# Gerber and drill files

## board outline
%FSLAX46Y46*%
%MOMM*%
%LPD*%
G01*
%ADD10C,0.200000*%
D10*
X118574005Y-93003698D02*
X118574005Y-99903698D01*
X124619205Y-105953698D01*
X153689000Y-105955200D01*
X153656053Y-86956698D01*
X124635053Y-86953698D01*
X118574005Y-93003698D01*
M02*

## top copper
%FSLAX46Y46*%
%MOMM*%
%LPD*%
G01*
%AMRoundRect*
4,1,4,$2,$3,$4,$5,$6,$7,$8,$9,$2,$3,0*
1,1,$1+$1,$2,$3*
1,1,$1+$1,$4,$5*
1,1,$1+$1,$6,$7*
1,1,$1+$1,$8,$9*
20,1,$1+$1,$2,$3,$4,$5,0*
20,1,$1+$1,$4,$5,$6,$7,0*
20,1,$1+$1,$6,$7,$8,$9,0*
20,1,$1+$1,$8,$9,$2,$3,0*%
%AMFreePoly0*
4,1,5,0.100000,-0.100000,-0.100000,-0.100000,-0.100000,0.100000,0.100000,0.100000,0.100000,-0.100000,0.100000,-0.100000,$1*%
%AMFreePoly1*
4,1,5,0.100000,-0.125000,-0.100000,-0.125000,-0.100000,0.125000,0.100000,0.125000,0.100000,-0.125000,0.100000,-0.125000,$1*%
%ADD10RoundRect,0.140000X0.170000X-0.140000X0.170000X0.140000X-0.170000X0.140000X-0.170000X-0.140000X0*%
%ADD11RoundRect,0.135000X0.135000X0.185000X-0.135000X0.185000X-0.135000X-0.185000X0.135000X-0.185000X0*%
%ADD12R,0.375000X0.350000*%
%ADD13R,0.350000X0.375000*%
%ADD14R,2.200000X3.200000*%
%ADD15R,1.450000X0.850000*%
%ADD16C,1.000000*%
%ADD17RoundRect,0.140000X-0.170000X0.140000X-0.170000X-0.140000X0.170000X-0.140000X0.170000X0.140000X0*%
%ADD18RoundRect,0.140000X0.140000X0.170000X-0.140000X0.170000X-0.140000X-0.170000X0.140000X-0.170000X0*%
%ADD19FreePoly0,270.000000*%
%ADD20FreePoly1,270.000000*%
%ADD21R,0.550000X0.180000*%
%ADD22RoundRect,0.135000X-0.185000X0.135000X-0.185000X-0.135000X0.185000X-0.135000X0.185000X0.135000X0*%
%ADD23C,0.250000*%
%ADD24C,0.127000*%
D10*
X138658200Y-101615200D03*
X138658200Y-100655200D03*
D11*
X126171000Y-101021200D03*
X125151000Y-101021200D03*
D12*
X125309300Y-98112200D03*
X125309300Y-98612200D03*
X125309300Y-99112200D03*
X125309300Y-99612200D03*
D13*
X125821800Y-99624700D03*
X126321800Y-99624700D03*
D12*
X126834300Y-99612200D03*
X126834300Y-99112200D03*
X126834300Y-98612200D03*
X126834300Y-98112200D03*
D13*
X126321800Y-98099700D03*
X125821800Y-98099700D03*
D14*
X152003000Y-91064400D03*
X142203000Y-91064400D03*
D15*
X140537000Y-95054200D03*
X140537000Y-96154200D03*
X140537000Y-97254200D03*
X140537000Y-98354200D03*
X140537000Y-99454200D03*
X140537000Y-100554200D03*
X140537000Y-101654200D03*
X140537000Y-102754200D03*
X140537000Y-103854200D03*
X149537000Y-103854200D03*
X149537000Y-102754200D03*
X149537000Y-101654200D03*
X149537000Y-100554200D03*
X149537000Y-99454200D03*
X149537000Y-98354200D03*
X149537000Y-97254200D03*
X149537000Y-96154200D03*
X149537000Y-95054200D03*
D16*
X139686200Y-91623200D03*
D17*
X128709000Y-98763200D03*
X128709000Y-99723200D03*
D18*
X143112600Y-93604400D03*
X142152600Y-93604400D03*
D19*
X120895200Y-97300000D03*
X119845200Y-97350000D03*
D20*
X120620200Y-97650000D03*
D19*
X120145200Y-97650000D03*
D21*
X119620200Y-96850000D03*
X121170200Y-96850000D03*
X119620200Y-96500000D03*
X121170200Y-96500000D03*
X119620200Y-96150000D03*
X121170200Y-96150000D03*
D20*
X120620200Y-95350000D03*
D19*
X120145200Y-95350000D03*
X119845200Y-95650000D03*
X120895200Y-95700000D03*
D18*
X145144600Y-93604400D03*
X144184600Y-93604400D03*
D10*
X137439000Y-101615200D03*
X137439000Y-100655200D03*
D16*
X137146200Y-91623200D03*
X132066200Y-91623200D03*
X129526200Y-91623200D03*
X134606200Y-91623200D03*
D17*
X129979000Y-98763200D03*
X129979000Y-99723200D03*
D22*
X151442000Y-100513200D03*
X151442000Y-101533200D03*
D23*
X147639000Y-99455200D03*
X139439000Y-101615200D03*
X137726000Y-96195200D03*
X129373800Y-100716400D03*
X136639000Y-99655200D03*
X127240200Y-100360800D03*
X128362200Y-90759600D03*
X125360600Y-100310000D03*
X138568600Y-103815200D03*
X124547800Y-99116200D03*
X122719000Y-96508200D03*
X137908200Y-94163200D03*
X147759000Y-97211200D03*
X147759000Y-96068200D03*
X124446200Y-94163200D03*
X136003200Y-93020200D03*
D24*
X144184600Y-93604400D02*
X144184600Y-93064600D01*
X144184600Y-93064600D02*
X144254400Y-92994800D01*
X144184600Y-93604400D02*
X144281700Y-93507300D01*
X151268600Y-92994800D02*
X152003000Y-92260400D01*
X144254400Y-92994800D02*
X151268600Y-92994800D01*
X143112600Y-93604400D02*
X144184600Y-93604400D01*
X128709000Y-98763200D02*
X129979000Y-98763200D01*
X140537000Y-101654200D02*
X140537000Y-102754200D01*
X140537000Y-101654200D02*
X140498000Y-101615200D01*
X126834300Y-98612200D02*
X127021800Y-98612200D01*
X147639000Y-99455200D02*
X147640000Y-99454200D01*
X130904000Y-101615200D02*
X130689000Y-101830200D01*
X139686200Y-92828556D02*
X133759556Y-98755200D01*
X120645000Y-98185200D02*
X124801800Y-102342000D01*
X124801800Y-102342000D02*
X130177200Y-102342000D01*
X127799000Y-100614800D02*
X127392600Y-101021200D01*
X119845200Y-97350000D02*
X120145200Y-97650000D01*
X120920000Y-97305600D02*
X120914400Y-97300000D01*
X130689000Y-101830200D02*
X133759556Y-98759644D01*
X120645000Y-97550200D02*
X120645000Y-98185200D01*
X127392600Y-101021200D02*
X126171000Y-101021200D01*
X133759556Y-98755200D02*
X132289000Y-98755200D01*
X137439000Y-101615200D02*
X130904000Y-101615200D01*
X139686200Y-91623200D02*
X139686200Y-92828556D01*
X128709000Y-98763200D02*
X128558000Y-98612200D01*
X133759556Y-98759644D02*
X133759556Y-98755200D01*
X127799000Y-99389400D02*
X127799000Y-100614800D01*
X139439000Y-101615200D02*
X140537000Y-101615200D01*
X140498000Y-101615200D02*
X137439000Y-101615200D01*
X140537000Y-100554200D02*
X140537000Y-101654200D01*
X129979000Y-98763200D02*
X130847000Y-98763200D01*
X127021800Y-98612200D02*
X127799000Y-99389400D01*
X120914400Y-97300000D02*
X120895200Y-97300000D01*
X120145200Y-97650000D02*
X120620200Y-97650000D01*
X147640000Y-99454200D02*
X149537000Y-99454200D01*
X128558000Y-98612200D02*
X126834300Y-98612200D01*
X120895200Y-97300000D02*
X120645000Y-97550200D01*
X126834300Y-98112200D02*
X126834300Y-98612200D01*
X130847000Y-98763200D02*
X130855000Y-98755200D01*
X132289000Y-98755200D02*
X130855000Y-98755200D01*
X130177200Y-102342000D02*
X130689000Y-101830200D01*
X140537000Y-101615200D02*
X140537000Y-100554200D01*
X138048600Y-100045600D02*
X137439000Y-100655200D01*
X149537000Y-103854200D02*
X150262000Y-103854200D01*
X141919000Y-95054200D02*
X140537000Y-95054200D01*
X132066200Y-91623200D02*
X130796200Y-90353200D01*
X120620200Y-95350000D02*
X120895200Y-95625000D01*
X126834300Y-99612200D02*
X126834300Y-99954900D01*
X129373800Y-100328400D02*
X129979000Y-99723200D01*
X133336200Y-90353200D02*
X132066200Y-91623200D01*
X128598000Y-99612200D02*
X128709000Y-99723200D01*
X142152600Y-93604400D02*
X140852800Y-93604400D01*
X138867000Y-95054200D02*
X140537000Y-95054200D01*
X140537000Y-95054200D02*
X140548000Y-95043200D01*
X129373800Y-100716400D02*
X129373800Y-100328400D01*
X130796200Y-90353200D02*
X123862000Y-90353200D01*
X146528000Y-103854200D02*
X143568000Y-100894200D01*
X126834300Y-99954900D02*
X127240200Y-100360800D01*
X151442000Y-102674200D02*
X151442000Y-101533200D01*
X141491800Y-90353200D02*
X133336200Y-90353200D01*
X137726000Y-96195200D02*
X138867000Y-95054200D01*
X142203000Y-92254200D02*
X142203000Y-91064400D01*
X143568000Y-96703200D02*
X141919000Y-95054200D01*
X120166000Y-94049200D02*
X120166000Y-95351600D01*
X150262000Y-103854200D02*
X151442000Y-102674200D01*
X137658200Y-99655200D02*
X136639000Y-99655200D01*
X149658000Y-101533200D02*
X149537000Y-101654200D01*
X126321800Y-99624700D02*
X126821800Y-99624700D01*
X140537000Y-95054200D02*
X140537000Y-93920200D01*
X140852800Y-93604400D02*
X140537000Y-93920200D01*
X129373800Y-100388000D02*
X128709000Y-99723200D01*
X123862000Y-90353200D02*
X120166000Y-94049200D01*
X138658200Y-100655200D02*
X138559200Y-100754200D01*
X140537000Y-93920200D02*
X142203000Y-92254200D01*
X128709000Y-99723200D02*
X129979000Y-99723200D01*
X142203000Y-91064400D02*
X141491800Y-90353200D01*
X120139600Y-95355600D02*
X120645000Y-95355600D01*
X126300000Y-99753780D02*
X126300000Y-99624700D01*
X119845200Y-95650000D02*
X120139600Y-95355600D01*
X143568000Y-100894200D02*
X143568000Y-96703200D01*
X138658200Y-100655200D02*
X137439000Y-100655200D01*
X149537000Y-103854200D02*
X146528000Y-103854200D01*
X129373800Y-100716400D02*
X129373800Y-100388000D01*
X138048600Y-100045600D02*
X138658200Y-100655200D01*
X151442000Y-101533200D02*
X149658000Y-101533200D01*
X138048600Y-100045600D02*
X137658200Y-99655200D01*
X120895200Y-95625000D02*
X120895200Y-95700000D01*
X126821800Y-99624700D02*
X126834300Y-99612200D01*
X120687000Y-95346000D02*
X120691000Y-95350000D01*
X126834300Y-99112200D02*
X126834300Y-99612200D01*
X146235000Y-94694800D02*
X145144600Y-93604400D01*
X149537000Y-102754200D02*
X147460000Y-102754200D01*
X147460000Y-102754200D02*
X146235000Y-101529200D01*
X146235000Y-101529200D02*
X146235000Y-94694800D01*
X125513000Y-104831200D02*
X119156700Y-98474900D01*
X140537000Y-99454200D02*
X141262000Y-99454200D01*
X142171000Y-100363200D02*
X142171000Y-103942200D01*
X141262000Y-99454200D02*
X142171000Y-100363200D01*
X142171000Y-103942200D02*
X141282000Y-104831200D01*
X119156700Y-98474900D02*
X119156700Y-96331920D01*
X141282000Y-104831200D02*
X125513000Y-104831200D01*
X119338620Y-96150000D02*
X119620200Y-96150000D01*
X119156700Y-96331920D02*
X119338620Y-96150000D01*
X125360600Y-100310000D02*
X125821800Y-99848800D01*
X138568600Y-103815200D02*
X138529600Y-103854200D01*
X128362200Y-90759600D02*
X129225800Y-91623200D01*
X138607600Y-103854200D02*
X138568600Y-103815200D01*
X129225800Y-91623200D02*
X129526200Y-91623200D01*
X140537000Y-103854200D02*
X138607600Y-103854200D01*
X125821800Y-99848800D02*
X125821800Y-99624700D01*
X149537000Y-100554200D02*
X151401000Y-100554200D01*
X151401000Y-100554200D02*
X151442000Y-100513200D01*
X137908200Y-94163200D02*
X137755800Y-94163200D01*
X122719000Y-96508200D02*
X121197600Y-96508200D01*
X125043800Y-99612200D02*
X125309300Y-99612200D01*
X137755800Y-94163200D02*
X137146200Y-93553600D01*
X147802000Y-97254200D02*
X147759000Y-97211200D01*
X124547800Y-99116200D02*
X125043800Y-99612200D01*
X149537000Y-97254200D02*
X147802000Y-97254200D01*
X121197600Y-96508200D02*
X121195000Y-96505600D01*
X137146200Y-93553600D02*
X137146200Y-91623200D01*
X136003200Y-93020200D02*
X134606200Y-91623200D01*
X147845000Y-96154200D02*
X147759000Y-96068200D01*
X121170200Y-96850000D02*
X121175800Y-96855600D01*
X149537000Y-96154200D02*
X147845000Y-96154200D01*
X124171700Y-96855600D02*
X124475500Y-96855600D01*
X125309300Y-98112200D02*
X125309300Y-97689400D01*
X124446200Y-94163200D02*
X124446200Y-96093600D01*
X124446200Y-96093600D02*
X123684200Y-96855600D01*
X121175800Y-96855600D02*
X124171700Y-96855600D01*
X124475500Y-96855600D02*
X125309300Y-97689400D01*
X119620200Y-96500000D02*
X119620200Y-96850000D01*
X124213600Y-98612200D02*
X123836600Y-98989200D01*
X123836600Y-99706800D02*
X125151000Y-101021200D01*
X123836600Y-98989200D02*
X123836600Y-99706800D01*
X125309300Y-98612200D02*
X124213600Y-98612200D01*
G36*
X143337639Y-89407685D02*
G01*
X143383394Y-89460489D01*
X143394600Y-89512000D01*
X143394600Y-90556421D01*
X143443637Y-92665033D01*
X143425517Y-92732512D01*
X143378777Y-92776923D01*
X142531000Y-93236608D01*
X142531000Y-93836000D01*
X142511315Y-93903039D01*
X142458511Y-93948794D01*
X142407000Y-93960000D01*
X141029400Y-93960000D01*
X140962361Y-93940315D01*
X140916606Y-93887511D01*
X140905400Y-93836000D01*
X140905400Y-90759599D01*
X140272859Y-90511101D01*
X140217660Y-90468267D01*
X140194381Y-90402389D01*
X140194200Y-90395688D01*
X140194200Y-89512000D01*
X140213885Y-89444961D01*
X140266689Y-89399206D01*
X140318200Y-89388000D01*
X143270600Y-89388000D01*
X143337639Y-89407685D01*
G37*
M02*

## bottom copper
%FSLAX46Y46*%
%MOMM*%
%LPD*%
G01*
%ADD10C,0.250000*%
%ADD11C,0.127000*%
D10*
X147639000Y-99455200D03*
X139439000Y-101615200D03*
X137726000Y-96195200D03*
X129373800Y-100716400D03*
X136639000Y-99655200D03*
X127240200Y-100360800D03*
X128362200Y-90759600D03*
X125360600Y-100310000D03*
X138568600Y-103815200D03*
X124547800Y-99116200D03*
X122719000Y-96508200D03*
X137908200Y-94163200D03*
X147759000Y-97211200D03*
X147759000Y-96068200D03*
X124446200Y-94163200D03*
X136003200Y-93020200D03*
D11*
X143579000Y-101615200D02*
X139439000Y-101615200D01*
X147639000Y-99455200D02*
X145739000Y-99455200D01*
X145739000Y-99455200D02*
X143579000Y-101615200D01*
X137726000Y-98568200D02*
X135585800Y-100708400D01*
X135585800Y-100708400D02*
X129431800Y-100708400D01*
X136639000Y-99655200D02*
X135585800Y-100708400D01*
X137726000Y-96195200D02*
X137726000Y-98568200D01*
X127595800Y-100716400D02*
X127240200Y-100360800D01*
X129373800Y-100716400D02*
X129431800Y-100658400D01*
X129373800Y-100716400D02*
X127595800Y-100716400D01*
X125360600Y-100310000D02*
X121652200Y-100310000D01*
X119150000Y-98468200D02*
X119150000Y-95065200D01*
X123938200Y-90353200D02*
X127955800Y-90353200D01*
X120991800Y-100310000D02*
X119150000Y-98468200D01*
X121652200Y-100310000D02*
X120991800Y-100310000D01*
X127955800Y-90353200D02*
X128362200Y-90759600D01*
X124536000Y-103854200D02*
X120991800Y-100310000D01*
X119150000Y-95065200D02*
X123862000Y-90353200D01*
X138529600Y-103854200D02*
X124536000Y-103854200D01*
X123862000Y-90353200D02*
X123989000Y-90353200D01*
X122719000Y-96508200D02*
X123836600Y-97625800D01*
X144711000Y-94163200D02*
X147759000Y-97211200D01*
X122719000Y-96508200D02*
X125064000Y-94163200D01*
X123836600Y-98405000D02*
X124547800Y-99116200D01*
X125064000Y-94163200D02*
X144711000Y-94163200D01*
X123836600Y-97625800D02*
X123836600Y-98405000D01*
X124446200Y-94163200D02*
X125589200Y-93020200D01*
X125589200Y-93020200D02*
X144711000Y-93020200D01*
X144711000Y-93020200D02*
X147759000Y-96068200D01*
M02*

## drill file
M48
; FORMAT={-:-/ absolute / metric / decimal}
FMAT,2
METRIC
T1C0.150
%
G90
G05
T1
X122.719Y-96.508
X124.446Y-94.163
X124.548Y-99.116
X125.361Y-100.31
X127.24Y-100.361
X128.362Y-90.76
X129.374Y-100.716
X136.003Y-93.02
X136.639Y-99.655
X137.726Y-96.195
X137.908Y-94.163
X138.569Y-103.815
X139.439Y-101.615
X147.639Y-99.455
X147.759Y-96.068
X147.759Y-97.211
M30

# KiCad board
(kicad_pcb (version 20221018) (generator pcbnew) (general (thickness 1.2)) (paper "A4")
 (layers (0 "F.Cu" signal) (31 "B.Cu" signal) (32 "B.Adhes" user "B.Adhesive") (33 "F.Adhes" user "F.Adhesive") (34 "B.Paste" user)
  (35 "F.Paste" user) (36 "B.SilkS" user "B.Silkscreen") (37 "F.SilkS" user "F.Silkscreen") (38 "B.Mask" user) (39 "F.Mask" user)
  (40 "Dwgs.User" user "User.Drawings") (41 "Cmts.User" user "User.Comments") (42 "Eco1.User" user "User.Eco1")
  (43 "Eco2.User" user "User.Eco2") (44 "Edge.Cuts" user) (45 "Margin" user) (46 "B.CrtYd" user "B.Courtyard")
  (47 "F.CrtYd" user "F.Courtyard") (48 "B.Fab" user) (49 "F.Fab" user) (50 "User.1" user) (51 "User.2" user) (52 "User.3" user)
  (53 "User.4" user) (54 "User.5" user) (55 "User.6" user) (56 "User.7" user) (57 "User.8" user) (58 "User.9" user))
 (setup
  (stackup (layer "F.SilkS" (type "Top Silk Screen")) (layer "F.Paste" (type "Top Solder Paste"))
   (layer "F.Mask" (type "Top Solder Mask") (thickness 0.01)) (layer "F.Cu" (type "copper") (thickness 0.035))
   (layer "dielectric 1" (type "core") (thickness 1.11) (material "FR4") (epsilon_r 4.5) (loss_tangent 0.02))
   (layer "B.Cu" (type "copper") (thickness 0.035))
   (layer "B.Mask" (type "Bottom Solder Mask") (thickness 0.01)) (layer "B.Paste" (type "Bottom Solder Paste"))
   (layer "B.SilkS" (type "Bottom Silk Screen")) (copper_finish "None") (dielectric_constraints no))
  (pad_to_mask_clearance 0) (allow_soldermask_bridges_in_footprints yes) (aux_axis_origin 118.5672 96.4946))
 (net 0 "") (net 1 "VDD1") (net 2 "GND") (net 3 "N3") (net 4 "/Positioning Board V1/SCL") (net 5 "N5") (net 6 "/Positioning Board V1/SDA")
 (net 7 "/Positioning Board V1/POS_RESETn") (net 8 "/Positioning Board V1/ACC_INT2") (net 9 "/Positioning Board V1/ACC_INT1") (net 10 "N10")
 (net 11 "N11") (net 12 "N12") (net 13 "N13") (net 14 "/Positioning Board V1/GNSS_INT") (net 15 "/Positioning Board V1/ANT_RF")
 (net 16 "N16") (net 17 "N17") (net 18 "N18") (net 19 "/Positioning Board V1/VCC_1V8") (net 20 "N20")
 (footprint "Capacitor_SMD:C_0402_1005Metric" (layer "F.Cu") (at 138.6582 101.1352 90)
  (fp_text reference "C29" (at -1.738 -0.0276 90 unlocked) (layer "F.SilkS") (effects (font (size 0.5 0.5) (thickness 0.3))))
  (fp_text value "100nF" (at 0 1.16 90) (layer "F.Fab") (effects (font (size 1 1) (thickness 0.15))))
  (pad "1" smd roundrect (at -0.48 0 90) (size 0.56 0.62) (layers "F.Cu" "F.Paste" "F.Mask") (roundrect_rratio 0.25) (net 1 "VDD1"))
  (pad "2" smd roundrect (at 0.48 0 90) (size 0.56 0.62) (layers "F.Cu" "F.Paste" "F.Mask") (roundrect_rratio 0.25) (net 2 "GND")))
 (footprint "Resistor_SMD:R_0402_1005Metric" (layer "F.Cu") (at 125.661 101.0212 180)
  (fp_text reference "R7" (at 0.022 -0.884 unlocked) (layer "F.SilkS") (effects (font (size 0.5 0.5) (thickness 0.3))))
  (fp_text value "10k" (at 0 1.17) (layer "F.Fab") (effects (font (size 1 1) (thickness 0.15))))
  (pad "1" smd roundrect (at -0.51 0 180) (size 0.54 0.64) (layers "F.Cu" "F.Paste" "F.Mask") (roundrect_rratio 0.25) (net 1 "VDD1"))
  (pad "2" smd roundrect (at 0.51 0 180) (size 0.54 0.64) (layers "F.Cu" "F.Paste" "F.Mask") (roundrect_rratio 0.25) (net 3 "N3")))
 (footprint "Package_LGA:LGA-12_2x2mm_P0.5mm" (layer "F.Cu") (at 126.0718 98.8622)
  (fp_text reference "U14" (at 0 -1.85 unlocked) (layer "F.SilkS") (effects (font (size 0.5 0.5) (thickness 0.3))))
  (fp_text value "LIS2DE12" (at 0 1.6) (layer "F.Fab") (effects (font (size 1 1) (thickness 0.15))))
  (pad "1" smd rect (at -0.7625 -0.75) (size 0.375 0.35) (layers "F.Cu" "F.Paste" "F.Mask") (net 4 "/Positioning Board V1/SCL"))
  (pad "2" smd rect (at -0.7625 -0.25) (size 0.375 0.35) (layers "F.Cu" "F.Paste" "F.Mask") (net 3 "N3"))
  (pad "3" smd rect (at -0.7625 0.25) (size 0.375 0.35) (layers "F.Cu" "F.Paste" "F.Mask") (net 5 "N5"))
  (pad "4" smd rect (at -0.7625 0.75) (size 0.375 0.35) (layers "F.Cu" "F.Paste" "F.Mask") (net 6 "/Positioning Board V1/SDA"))
  (pad "5" smd rect (at -0.25 0.7625 90) (size 0.375 0.35) (layers "F.Cu" "F.Paste" "F.Mask") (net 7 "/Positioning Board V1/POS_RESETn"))
  (pad "6" smd rect (at 0.25 0.7625 90) (size 0.375 0.35) (layers "F.Cu" "F.Paste" "F.Mask") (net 2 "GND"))
  (pad "7" smd rect (at 0.7625 0.75) (size 0.375 0.35) (layers "F.Cu" "F.Paste" "F.Mask") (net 2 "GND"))
  (pad "8" smd rect (at 0.7625 0.25) (size 0.375 0.35) (layers "F.Cu" "F.Paste" "F.Mask") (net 2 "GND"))
  (pad "9" smd rect (at 0.7625 -0.25) (size 0.375 0.35) (layers "F.Cu" "F.Paste" "F.Mask") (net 1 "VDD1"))
  (pad "10" smd rect (at 0.7625 -0.75) (size 0.375 0.35) (layers "F.Cu" "F.Paste" "F.Mask") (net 1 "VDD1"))
  (pad "11" smd rect (at 0.25 -0.7625 90) (size 0.375 0.35) (layers "F.Cu" "F.Paste" "F.Mask") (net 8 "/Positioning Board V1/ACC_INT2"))
  (pad "12" smd rect (at -0.25 -0.7625 90) (size 0.375 0.35) (layers "F.Cu" "F.Paste" "F.Mask") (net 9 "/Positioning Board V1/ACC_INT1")))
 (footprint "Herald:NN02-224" (layer "F.Cu") (at 147.103 91.0644 180)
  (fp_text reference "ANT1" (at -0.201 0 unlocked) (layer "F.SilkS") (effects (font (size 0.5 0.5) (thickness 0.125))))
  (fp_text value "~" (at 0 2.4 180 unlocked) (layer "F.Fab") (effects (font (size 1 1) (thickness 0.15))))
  (pad "1" smd rect (at -4.9 0 180) (size 2.2 3.2) (layers "F.Cu" "F.Paste" "F.Mask") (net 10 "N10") (thermal_bridge_angle 45))
  (pad "2" smd rect (at 4.9 0 180) (size 2.2 3.2) (layers "F.Cu" "F.Paste" "F.Mask") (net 2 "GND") (thermal_bridge_angle 45)))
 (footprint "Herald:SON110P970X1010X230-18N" (layer "F.Cu") (at 145.037 99.4542)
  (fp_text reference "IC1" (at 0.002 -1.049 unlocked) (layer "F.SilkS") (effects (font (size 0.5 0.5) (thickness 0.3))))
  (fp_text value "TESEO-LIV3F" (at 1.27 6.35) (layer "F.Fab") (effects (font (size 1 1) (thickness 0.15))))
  (pad "1" smd rect (at -4.5 -4.4) (size 1.45 0.85) (layers "F.Cu" "F.Paste" "F.Mask") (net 2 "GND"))
  (pad "2" smd rect (at -4.5 -3.3) (size 1.45 0.85) (layers "F.Cu" "F.Paste" "F.Mask") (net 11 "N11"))
  (pad "3" smd rect (at -4.5 -2.2) (size 1.45 0.85) (layers "F.Cu" "F.Paste" "F.Mask") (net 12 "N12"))
  (pad "4" smd rect (at -4.5 -1.1) (size 1.45 0.85) (layers "F.Cu" "F.Paste" "F.Mask") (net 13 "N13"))
  (pad "5" smd rect (at -4.5 0) (size 1.45 0.85) (layers "F.Cu" "F.Paste" "F.Mask") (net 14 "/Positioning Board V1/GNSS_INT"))
  (pad "6" smd rect (at -4.5 1.1) (size 1.45 0.85) (layers "F.Cu" "F.Paste" "F.Mask") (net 1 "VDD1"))
  (pad "7" smd rect (at -4.5 2.2) (size 1.45 0.85) (layers "F.Cu" "F.Paste" "F.Mask") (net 1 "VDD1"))
  (pad "8" smd rect (at -4.5 3.3) (size 1.45 0.85) (layers "F.Cu" "F.Paste" "F.Mask") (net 1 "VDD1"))
  (pad "9" smd rect (at -4.5 4.4) (size 1.45 0.85) (layers "F.Cu" "F.Paste" "F.Mask") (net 7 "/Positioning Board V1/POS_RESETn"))
  (pad "10" smd rect (at 4.5 4.4) (size 1.45 0.85) (layers "F.Cu" "F.Paste" "F.Mask") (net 2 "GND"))
  (pad "11" smd rect (at 4.5 3.3) (size 1.45 0.85) (layers "F.Cu" "F.Paste" "F.Mask") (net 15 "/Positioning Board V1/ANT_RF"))
  (pad "12" smd rect (at 4.5 2.2) (size 1.45 0.85) (layers "F.Cu" "F.Paste" "F.Mask") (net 2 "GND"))
  (pad "13" smd rect (at 4.5 1.1) (size 1.45 0.85) (layers "F.Cu" "F.Paste" "F.Mask") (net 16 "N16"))
  (pad "14" smd rect (at 4.5 0) (size 1.45 0.85) (layers "F.Cu" "F.Paste" "F.Mask") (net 1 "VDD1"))
  (pad "15" smd rect (at 4.5 -1.1) (size 1.45 0.85) (layers "F.Cu" "F.Paste" "F.Mask") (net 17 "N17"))
  (pad "16" smd rect (at 4.5 -2.2) (size 1.45 0.85) (layers "F.Cu" "F.Paste" "F.Mask") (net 6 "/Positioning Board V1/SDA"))
  (pad "17" smd rect (at 4.5 -3.3) (size 1.45 0.85) (layers "F.Cu" "F.Paste" "F.Mask") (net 4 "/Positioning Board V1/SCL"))
  (pad "18" smd rect (at 4.5 -4.4) (size 1.45 0.85) (layers "F.Cu" "F.Paste" "F.Mask") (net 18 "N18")))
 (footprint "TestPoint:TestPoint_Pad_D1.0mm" (layer "F.Cu") (at 139.6862 91.6232)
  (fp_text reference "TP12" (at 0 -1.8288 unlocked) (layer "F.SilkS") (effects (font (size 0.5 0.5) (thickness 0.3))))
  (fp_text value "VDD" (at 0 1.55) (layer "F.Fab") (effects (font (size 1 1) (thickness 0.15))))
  (pad "1" smd circle (at 0 0) (size 1 1) (layers "F.Cu" "F.Mask") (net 1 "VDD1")))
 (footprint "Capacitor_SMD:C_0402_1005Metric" (layer "F.Cu") (at 128.709 99.2432 -90)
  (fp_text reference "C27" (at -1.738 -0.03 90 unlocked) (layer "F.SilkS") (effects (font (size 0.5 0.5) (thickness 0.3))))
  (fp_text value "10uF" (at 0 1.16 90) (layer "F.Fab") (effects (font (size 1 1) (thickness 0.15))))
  (pad "1" smd roundrect (at -0.48 0 270) (size 0.56 0.62) (layers "F.Cu" "F.Paste" "F.Mask") (roundrect_rratio 0.25) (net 1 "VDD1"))
  (pad "2" smd roundrect (at 0.48 0 270) (size 0.56 0.62) (layers "F.Cu" "F.Paste" "F.Mask") (roundrect_rratio 0.25) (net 2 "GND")))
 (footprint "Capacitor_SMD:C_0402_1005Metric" (layer "F.Cu") (at 142.6326 93.6044 180)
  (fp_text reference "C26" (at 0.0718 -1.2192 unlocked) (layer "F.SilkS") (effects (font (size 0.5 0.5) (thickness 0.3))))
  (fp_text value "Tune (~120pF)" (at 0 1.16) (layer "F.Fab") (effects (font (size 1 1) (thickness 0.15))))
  (pad "1" smd roundrect (at -0.48 0 180) (size 0.56 0.62) (layers "F.Cu" "F.Paste" "F.Mask") (roundrect_rratio 0.25) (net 10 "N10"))
  (pad "2" smd roundrect (at 0.48 0 180) (size 0.56 0.62) (layers "F.Cu" "F.Paste" "F.Mask") (roundrect_rratio 0.25) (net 2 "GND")))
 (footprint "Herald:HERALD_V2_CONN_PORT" (layer "F.Cu") (at 120.3952 96.5 -90)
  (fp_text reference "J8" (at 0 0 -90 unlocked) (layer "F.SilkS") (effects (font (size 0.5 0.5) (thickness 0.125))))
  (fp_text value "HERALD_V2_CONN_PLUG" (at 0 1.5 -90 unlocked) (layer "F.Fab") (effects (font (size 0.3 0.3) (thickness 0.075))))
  (pad "1" smd custom (at 0.8 -0.5 270) (size 0.2 0.2) (layers "F.Cu" "F.Paste" "F.Mask") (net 1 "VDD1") (thermal_bridge_angle 45)
   (options (clearance outline) (anchor rect)) (primitives))
  (pad "1" smd custom (at 0.85 0.55 270) (size 0.2 0.2) (layers "F.Cu" "F.Paste" "F.Mask") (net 1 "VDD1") (thermal_bridge_angle 45)
   (options (clearance outline) (anchor rect)) (primitives))
  (pad "1" smd custom (at 1.15 -0.225 270) (size 0.2 0.25) (layers "F.Cu" "F.Paste" "F.Mask") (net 1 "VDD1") (thermal_bridge_angle 45)
   (options (clearance outline) (anchor rect)) (primitives))
  (pad "1" smd custom (at 1.15 0.25 270) (size 0.2 0.2) (layers "F.Cu" "F.Paste" "F.Mask") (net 1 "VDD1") (thermal_bridge_angle 45)
   (options (clearance outline) (anchor rect)) (primitives))
  (pad "2" smd rect (at 0.35 0.775 270) (size 0.18 0.55) (layers "F.Cu" "F.Paste" "F.Mask") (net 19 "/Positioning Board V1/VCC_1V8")
   (thermal_bridge_angle 45))
  (pad "3" smd rect (at 0.35 -0.775 270) (size 0.18 0.55) (layers "F.Cu" "F.Paste" "F.Mask") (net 4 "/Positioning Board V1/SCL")
   (thermal_bridge_angle 45))
  (pad "4" smd rect (at 0 0.775 270) (size 0.18 0.55) (layers "F.Cu" "F.Paste" "F.Mask") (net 19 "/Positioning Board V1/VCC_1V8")
   (thermal_bridge_angle 45))
  (pad "5" smd rect (at 0 -0.775 270) (size 0.18 0.55) (layers "F.Cu" "F.Paste" "F.Mask") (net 6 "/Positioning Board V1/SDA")
   (thermal_bridge_angle 45))
  (pad "6" smd rect (at -0.35 0.775 270) (size 0.18 0.55) (layers "F.Cu" "F.Paste" "F.Mask") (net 14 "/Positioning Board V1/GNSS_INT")
   (thermal_bridge_angle 45))
  (pad "7" smd rect (at -0.35 -0.775 270) (size 0.18 0.55) (layers "F.Cu" "F.Paste" "F.Mask") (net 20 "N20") (thermal_bridge_angle 45))
  (pad "8" smd custom (at -1.15 -0.225 270) (size 0.2 0.25) (layers "F.Cu" "F.Paste" "F.Mask") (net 2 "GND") (thermal_bridge_angle 45)
   (options (clearance outline) (anchor rect)) (primitives))
  (pad "8" smd custom (at -1.15 0.25 270) (size 0.2 0.2) (layers "F.Cu" "F.Paste" "F.Mask") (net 2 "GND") (thermal_bridge_angle 45)
   (options (clearance outline) (anchor rect)) (primitives))
  (pad "8" smd custom (at -0.85 0.55 270) (size 0.2 0.2) (layers "F.Cu" "F.Paste" "F.Mask") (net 2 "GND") (thermal_bridge_angle 45)
   (options (clearance outline) (anchor rect)) (primitives))
  (pad "8" smd custom (at -0.8 -0.5 270) (size 0.2 0.2) (layers "F.Cu" "F.Paste" "F.Mask") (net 2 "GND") (thermal_bridge_angle 45)
   (options (clearance outline) (anchor rect)) (primitives)))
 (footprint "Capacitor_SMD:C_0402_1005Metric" (layer "F.Cu") (at 144.6646 93.6044 180)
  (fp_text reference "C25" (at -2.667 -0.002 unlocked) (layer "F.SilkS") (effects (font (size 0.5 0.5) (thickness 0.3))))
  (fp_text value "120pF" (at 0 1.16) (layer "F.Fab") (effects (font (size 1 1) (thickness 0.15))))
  (pad "1" smd roundrect (at -0.48 0 180) (size 0.56 0.62) (layers "F.Cu" "F.Paste" "F.Mask") (roundrect_rratio 0.25)
   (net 15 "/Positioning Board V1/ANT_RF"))
  (pad "2" smd roundrect (at 0.48 0 180) (size 0.56 0.62) (layers "F.Cu" "F.Paste" "F.Mask") (roundrect_rratio 0.25) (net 10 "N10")))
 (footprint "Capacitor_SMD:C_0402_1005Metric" (layer "F.Cu") (at 137.439 101.1352 90)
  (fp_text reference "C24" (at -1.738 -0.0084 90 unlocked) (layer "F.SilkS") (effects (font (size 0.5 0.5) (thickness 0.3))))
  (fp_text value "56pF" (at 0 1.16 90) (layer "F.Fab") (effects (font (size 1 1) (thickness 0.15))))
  (pad "1" smd roundrect (at -0.48 0 90) (size 0.56 0.62) (layers "F.Cu" "F.Paste" "F.Mask") (roundrect_rratio 0.25) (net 1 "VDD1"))
  (pad "2" smd roundrect (at 0.48 0 90) (size 0.56 0.62) (layers "F.Cu" "F.Paste" "F.Mask") (roundrect_rratio 0.25) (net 2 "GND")))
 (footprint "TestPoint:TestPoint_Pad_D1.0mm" (layer "F.Cu") (at 137.1462 91.6232)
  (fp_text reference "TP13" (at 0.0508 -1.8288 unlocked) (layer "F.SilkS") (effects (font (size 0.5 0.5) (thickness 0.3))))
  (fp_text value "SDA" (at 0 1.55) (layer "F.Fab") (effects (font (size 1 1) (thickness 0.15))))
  (pad "1" smd circle (at 0 0) (size 1 1) (layers "F.Cu" "F.Mask") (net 6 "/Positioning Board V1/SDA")))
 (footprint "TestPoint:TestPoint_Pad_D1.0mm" (layer "F.Cu") (at 132.0662 91.6232)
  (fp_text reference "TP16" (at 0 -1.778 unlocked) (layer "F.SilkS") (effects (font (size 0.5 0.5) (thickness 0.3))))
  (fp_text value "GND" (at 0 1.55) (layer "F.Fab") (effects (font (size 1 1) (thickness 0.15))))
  (pad "1" smd circle (at 0 0) (size 1 1) (layers "F.Cu" "F.Mask") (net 2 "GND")))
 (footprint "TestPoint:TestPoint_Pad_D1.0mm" (layer "F.Cu") (at 129.5262 91.6232)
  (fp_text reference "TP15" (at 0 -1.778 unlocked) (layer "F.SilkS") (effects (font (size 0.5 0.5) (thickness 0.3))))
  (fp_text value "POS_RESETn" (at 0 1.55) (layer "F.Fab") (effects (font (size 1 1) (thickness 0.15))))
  (pad "1" smd circle (at 0 0) (size 1 1) (layers "F.Cu" "F.Mask") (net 7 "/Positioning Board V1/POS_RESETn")))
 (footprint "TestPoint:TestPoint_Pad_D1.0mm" (layer "F.Cu") (at 134.6062 91.6232)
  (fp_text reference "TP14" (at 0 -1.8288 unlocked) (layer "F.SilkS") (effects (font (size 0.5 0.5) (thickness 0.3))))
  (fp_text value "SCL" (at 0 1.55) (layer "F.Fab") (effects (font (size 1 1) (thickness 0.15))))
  (pad "1" smd circle (at 0 0) (size 1 1) (layers "F.Cu" "F.Mask") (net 4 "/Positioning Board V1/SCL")))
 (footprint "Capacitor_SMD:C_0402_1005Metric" (layer "F.Cu") (at 129.979 99.2432 -90)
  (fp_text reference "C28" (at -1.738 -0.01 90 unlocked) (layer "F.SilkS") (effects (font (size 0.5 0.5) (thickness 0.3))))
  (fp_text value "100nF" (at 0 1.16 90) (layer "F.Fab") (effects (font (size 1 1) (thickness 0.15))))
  (pad "1" smd roundrect (at -0.48 0 270) (size 0.56 0.62) (layers "F.Cu" "F.Paste" "F.Mask") (roundrect_rratio 0.25) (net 1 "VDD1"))
  (pad "2" smd roundrect (at 0.48 0 270) (size 0.56 0.62) (layers "F.Cu" "F.Paste" "F.Mask") (roundrect_rratio 0.25) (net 2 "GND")))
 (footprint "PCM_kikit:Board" (layer "F.Cu") (at 123.3286 88.118)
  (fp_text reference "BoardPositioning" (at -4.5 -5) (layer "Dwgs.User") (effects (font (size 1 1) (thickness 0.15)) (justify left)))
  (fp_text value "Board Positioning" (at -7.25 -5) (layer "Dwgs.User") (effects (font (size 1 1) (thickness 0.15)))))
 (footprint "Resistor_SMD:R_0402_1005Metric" (layer "F.Cu") (at 151.442 101.0232 -90)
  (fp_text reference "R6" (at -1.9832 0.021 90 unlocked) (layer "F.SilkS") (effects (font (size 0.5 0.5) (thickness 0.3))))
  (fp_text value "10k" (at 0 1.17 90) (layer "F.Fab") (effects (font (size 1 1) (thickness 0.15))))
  (pad "1" smd roundrect (at -0.51 0 270) (size 0.54 0.64) (layers "F.Cu" "F.Paste" "F.Mask") (roundrect_rratio 0.25) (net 16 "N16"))
  (pad "2" smd roundrect (at 0.51 0 270) (size 0.54 0.64) (layers "F.Cu" "F.Paste" "F.Mask") (roundrect_rratio 0.25) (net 2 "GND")))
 (gr_poly
  (pts (xy 118.574005 93.003698) (xy 118.574005 99.903698) (xy 124.619205 105.953698) (xy 153.689 105.9552) (xy 153.656053 86.956698)
   (xy 124.635053 86.953698))
  (stroke (width 0.2) (type solid)) (fill none) (layer "Edge.Cuts"))
 (segment (start 144.1846 93.6044) (end 144.1846 93.0646) (width 0.127) (layer "F.Cu") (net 10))
 (segment (start 144.1846 93.0646) (end 144.2544 92.9948) (width 0.127) (layer "F.Cu") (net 10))
 (segment (start 144.1846 93.6044) (end 144.2817 93.5073) (width 0.127) (layer "F.Cu") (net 10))
 (segment (start 151.2686 92.9948) (end 152.003 92.2604) (width 0.127) (layer "F.Cu") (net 10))
 (segment (start 144.2544 92.9948) (end 151.2686 92.9948) (width 0.127) (layer "F.Cu") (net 10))
 (segment (start 143.1126 93.6044) (end 144.1846 93.6044) (width 0.127) (layer "F.Cu") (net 10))
 (segment (start 128.709 98.7632) (end 129.979 98.7632) (width 0.127) (layer "F.Cu") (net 1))
 (segment (start 140.537 101.6542) (end 140.537 102.7542) (width 0.127) (layer "F.Cu") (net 1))
 (segment (start 140.537 101.6542) (end 140.498 101.6152) (width 0.127) (layer "F.Cu") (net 1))
 (segment (start 126.8343 98.6122) (end 127.0218 98.6122) (width 0.127) (layer "F.Cu") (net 1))
 (segment (start 147.639 99.4552) (end 147.64 99.4542) (width 0.127) (layer "F.Cu") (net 1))
 (segment (start 130.904 101.6152) (end 130.689 101.8302) (width 0.127) (layer "F.Cu") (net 1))
 (segment (start 139.6862 92.828556) (end 133.759556 98.7552) (width 0.127) (layer "F.Cu") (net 1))
 (segment (start 120.645 98.1852) (end 124.8018 102.342) (width 0.127) (layer "F.Cu") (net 1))
 (segment (start 124.8018 102.342) (end 130.1772 102.342) (width 0.127) (layer "F.Cu") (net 1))
 (segment (start 127.799 100.6148) (end 127.3926 101.0212) (width 0.127) (layer "F.Cu") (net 1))
 (segment (start 119.8452 97.35) (end 120.1452 97.65) (width 0.127) (layer "F.Cu") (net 1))
 (segment (start 120.92 97.3056) (end 120.9144 97.3) (width 0.127) (layer "F.Cu") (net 1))
 (segment (start 130.689 101.8302) (end 133.759556 98.759644) (width 0.127) (layer "F.Cu") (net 1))
 (segment (start 120.645 97.5502) (end 120.645 98.1852) (width 0.127) (layer "F.Cu") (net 1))
 (segment (start 127.3926 101.0212) (end 126.171 101.0212) (width 0.127) (layer "F.Cu") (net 1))
 (segment (start 133.759556 98.7552) (end 132.289 98.7552) (width 0.127) (layer "F.Cu") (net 1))
 (segment (start 137.439 101.6152) (end 130.904 101.6152) (width 0.127) (layer "F.Cu") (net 1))
 (segment (start 139.6862 91.6232) (end 139.6862 92.828556) (width 0.127) (layer "F.Cu") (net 1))
 (segment (start 128.709 98.7632) (end 128.558 98.6122) (width 0.127) (layer "F.Cu") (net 1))
 (segment (start 133.759556 98.759644) (end 133.759556 98.7552) (width 0.127) (layer "F.Cu") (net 1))
 (segment (start 127.799 99.3894) (end 127.799 100.6148) (width 0.127) (layer "F.Cu") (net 1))
 (segment (start 139.439 101.6152) (end 140.537 101.6152) (width 0.127) (layer "F.Cu") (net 1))
 (segment (start 140.498 101.6152) (end 137.439 101.6152) (width 0.127) (layer "F.Cu") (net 1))
 (segment (start 140.537 100.5542) (end 140.537 101.6542) (width 0.127) (layer "F.Cu") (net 1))
 (segment (start 129.979 98.7632) (end 130.847 98.7632) (width 0.127) (layer "F.Cu") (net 1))
 (segment (start 127.0218 98.6122) (end 127.799 99.3894) (width 0.127) (layer "F.Cu") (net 1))
 (segment (start 120.9144 97.3) (end 120.8952 97.3) (width 0.127) (layer "F.Cu") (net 1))
 (segment (start 120.1452 97.65) (end 120.6202 97.65) (width 0.127) (layer "F.Cu") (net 1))
 (segment (start 147.64 99.4542) (end 149.537 99.4542) (width 0.127) (layer "F.Cu") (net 1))
 (segment (start 128.558 98.6122) (end 126.8343 98.6122) (width 0.127) (layer "F.Cu") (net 1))
 (segment (start 120.8952 97.3) (end 120.645 97.5502) (width 0.127) (layer "F.Cu") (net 1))
 (segment (start 126.8343 98.1122) (end 126.8343 98.6122) (width 0.127) (layer "F.Cu") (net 1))
 (segment (start 130.847 98.7632) (end 130.855 98.7552) (width 0.127) (layer "F.Cu") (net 1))
 (segment (start 132.289 98.7552) (end 130.855 98.7552) (width 0.127) (layer "F.Cu") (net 1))
 (segment (start 130.1772 102.342) (end 130.689 101.8302) (width 0.127) (layer "F.Cu") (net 1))
 (segment (start 140.537 101.6152) (end 140.537 100.5542) (width 0.127) (layer "F.Cu") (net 1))
 (via (at 147.639 99.4552) (size 0.25) (drill 0.15) (layers "F.Cu" "B.Cu") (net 1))
 (via (at 139.439 101.6152) (size 0.25) (drill 0.15) (layers "F.Cu" "B.Cu") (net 1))
 (segment (start 143.579 101.6152) (end 139.439 101.6152) (width 0.127) (layer "B.Cu") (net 1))
 (segment (start 147.639 99.4552) (end 145.739 99.4552) (width 0.127) (layer "B.Cu") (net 1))
 (segment (start 145.739 99.4552) (end 143.579 101.6152) (width 0.127) (layer "B.Cu") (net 1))
 (segment (start 138.0486 100.0456) (end 137.439 100.6552) (width 0.127) (layer "F.Cu") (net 2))
 (segment (start 149.537 103.8542) (end 150.262 103.8542) (width 0.127) (layer "F.Cu") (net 2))
 (segment (start 141.919 95.0542) (end 140.537 95.0542) (width 0.127) (layer "F.Cu") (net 2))
 (segment (start 132.0662 91.6232) (end 130.7962 90.3532) (width 0.127) (layer "F.Cu") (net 2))
 (segment (start 120.6202 95.35) (end 120.8952 95.625) (width 0.127) (layer "F.Cu") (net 2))
 (segment (start 126.8343 99.6122) (end 126.8343 99.9549) (width 0.127) (layer "F.Cu") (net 2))
 (segment (start 129.3738 100.3284) (end 129.979 99.7232) (width 0.127) (layer "F.Cu") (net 2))
 (segment (start 133.3362 90.3532) (end 132.0662 91.6232) (width 0.127) (layer "F.Cu") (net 2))
 (segment (start 128.598 99.6122) (end 128.709 99.7232) (width 0.127) (layer "F.Cu") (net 2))
 (segment (start 142.1526 93.6044) (end 140.8528 93.6044) (width 0.127) (layer "F.Cu") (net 2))
 (segment (start 138.867 95.0542) (end 140.537 95.0542) (width 0.127) (layer "F.Cu") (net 2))
 (segment (start 140.537 95.0542) (end 140.548 95.0432) (width 0.127) (layer "F.Cu") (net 2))
 (segment (start 129.3738 100.7164) (end 129.3738 100.3284) (width 0.127) (layer "F.Cu") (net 2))
 (segment (start 130.7962 90.3532) (end 123.862 90.3532) (width 0.127) (layer "F.Cu") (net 2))
 (segment (start 146.528 103.8542) (end 143.568 100.8942) (width 0.127) (layer "F.Cu") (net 2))
 (segment (start 126.8343 99.9549) (end 127.2402 100.3608) (width 0.127) (layer "F.Cu") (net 2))
 (segment (start 151.442 102.6742) (end 151.442 101.5332) (width 0.127) (layer "F.Cu") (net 2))
 (segment (start 141.4918 90.3532) (end 133.3362 90.3532) (width 0.127) (layer "F.Cu") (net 2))
 (segment (start 137.726 96.1952) (end 138.867 95.0542) (width 0.127) (layer "F.Cu") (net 2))
 (segment (start 142.203 92.2542) (end 142.203 91.0644) (width 0.127) (layer "F.Cu") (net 2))
 (segment (start 143.568 96.7032) (end 141.919 95.0542) (width 0.127) (layer "F.Cu") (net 2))
 (segment (start 120.166 94.0492) (end 120.166 95.3516) (width 0.127) (layer "F.Cu") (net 2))
 (segment (start 150.262 103.8542) (end 151.442 102.6742) (width 0.127) (layer "F.Cu") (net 2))
 (segment (start 137.6582 99.6552) (end 136.639 99.6552) (width 0.127) (layer "F.Cu") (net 2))
 (segment (start 149.658 101.5332) (end 149.537 101.6542) (width 0.127) (layer "F.Cu") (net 2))
 (segment (start 126.3218 99.6247) (end 126.8218 99.6247) (width 0.127) (layer "F.Cu") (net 2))
 (segment (start 140.537 95.0542) (end 140.537 93.9202) (width 0.127) (layer "F.Cu") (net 2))
 (segment (start 140.8528 93.6044) (end 140.537 93.9202) (width 0.127) (layer "F.Cu") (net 2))
 (segment (start 129.3738 100.388) (end 128.709 99.7232) (width 0.127) (layer "F.Cu") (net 2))
 (segment (start 123.862 90.3532) (end 120.166 94.0492) (width 0.127) (layer "F.Cu") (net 2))
 (segment (start 138.6582 100.6552) (end 138.5592 100.7542) (width 0.127) (layer "F.Cu") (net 2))
 (segment (start 140.537 93.9202) (end 142.203 92.2542) (width 0.127) (layer "F.Cu") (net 2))
 (segment (start 128.709 99.7232) (end 129.979 99.7232) (width 0.127) (layer "F.Cu") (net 2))
 (segment (start 142.203 91.0644) (end 141.4918 90.3532) (width 0.127) (layer "F.Cu") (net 2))
 (segment (start 120.1396 95.3556) (end 120.645 95.3556) (width 0.127) (layer "F.Cu") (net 2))
 (segment (start 126.3 99.75378) (end 126.3 99.6247) (width 0.127) (layer "F.Cu") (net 2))
 (segment (start 119.8452 95.65) (end 120.1396 95.3556) (width 0.127) (layer "F.Cu") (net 2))
 (segment (start 143.568 100.8942) (end 143.568 96.7032) (width 0.127) (layer "F.Cu") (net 2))
 (segment (start 138.6582 100.6552) (end 137.439 100.6552) (width 0.127) (layer "F.Cu") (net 2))
 (segment (start 149.537 103.8542) (end 146.528 103.8542) (width 0.127) (layer "F.Cu") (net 2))
 (segment (start 129.3738 100.7164) (end 129.3738 100.388) (width 0.127) (layer "F.Cu") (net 2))
 (segment (start 138.0486 100.0456) (end 138.6582 100.6552) (width 0.127) (layer "F.Cu") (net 2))
 (segment (start 151.442 101.5332) (end 149.658 101.5332) (width 0.127) (layer "F.Cu") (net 2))
 (segment (start 138.0486 100.0456) (end 137.6582 99.6552) (width 0.127) (layer "F.Cu") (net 2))
 (segment (start 120.8952 95.625) (end 120.8952 95.7) (width 0.127) (layer "F.Cu") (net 2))
 (segment (start 126.8218 99.6247) (end 126.8343 99.6122) (width 0.127) (layer "F.Cu") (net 2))
 (segment (start 120.687 95.346) (end 120.691 95.35) (width 0.127) (layer "F.Cu") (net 2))
 (segment (start 126.8343 99.1122) (end 126.8343 99.6122) (width 0.127) (layer "F.Cu") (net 2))
 (via (at 137.726 96.1952) (size 0.25) (drill 0.15) (layers "F.Cu" "B.Cu") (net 2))
 (via (at 129.3738 100.7164) (size 0.25) (drill 0.15) (layers "F.Cu" "B.Cu") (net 2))
 (via (at 136.639 99.6552) (size 0.25) (drill 0.15) (layers "F.Cu" "B.Cu") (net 2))
 (via (at 127.2402 100.3608) (size 0.25) (drill 0.15) (layers "F.Cu" "B.Cu") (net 2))
 (segment (start 137.726 98.5682) (end 135.5858 100.7084) (width 0.127) (layer "B.Cu") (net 2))
 (segment (start 135.5858 100.7084) (end 129.4318 100.7084) (width 0.127) (layer "B.Cu") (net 2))
 (segment (start 136.639 99.6552) (end 135.5858 100.7084) (width 0.127) (layer "B.Cu") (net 2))
 (segment (start 137.726 96.1952) (end 137.726 98.5682) (width 0.127) (layer "B.Cu") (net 2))
 (segment (start 127.5958 100.7164) (end 127.2402 100.3608) (width 0.127) (layer "B.Cu") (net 2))
 (segment (start 129.3738 100.7164) (end 129.4318 100.6584) (width 0.127) (layer "B.Cu") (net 2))
 (segment (start 129.3738 100.7164) (end 127.5958 100.7164) (width 0.127) (layer "B.Cu") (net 2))
 (segment (start 146.235 94.6948) (end 145.1446 93.6044) (width 0.127) (layer "F.Cu") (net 15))
 (segment (start 149.537 102.7542) (end 147.46 102.7542) (width 0.127) (layer "F.Cu") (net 15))
 (segment (start 147.46 102.7542) (end 146.235 101.5292) (width 0.127) (layer "F.Cu") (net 15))
 (segment (start 146.235 101.5292) (end 146.235 94.6948) (width 0.127) (layer "F.Cu") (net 15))
 (segment (start 125.513 104.8312) (end 119.1567 98.4749) (width 0.127) (layer "F.Cu") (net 14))
 (segment (start 140.537 99.4542) (end 141.262 99.4542) (width 0.127) (layer "F.Cu") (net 14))
 (segment (start 142.171 100.3632) (end 142.171 103.9422) (width 0.127) (layer "F.Cu") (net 14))
 (segment (start 141.262 99.4542) (end 142.171 100.3632) (width 0.127) (layer "F.Cu") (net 14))
 (segment (start 142.171 103.9422) (end 141.282 104.8312) (width 0.127) (layer "F.Cu") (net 14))
 (segment (start 119.1567 98.4749) (end 119.1567 96.33192) (width 0.127) (layer "F.Cu") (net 14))
 (segment (start 141.282 104.8312) (end 125.513 104.8312) (width 0.127) (layer "F.Cu") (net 14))
 (segment (start 119.33862 96.15) (end 119.6202 96.15) (width 0.127) (layer "F.Cu") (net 14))
 (segment (start 119.1567 96.33192) (end 119.33862 96.15) (width 0.127) (layer "F.Cu") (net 14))
 (segment (start 125.3606 100.31) (end 125.8218 99.8488) (width 0.127) (layer "F.Cu") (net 7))
 (segment (start 138.5686 103.8152) (end 138.5296 103.8542) (width 0.127) (layer "F.Cu") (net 7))
 (segment (start 128.3622 90.7596) (end 129.2258 91.6232) (width 0.127) (layer "F.Cu") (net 7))
 (segment (start 138.6076 103.8542) (end 138.5686 103.8152) (width 0.127) (layer "F.Cu") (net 7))
 (segment (start 129.2258 91.6232) (end 129.5262 91.6232) (width 0.127) (layer "F.Cu") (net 7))
 (segment (start 140.537 103.8542) (end 138.6076 103.8542) (width 0.127) (layer "F.Cu") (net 7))
 (segment (start 125.8218 99.8488) (end 125.8218 99.6247) (width 0.127) (layer "F.Cu") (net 7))
 (via (at 128.3622 90.7596) (size 0.25) (drill 0.15) (layers "F.Cu" "B.Cu") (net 7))
 (via (at 125.3606 100.31) (size 0.25) (drill 0.15) (layers "F.Cu" "B.Cu") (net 7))
 (via (at 138.5686 103.8152) (size 0.25) (drill 0.15) (layers "F.Cu" "B.Cu") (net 7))
 (segment (start 125.3606 100.31) (end 121.6522 100.31) (width 0.127) (layer "B.Cu") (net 7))
 (segment (start 119.15 98.4682) (end 119.15 95.0652) (width 0.127) (layer "B.Cu") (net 7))
 (segment (start 123.9382 90.3532) (end 127.9558 90.3532) (width 0.127) (layer "B.Cu") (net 7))
 (segment (start 120.9918 100.31) (end 119.15 98.4682) (width 0.127) (layer "B.Cu") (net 7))
 (segment (start 121.6522 100.31) (end 120.9918 100.31) (width 0.127) (layer "B.Cu") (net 7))
 (segment (start 127.9558 90.3532) (end 128.3622 90.7596) (width 0.127) (layer "B.Cu") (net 7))
 (segment (start 124.536 103.8542) (end 120.9918 100.31) (width 0.127) (layer "B.Cu") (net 7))
 (segment (start 119.15 95.0652) (end 123.862 90.3532) (width 0.127) (layer "B.Cu") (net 7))
 (segment (start 138.5296 103.8542) (end 124.536 103.8542) (width 0.127) (layer "B.Cu") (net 7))
 (segment (start 123.862 90.3532) (end 123.989 90.3532) (width 0.127) (layer "B.Cu") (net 7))
 (segment (start 149.537 100.5542) (end 151.401 100.5542) (width 0.127) (layer "F.Cu") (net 16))
 (segment (start 151.401 100.5542) (end 151.442 100.5132) (width 0.127) (layer "F.Cu") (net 16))
 (segment (start 137.9082 94.1632) (end 137.7558 94.1632) (width 0.127) (layer "F.Cu") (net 6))
 (segment (start 122.719 96.5082) (end 121.1976 96.5082) (width 0.127) (layer "F.Cu") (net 6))
 (segment (start 125.0438 99.6122) (end 125.3093 99.6122) (width 0.127) (layer "F.Cu") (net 6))
 (segment (start 137.7558 94.1632) (end 137.1462 93.5536) (width 0.127) (layer "F.Cu") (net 6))
 (segment (start 147.802 97.2542) (end 147.759 97.2112) (width 0.127) (layer "F.Cu") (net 6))
 (segment (start 124.5478 99.1162) (end 125.0438 99.6122) (width 0.127) (layer "F.Cu") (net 6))
 (segment (start 149.537 97.2542) (end 147.802 97.2542) (width 0.127) (layer "F.Cu") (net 6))
 (segment (start 121.1976 96.5082) (end 121.195 96.5056) (width 0.127) (layer "F.Cu") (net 6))
 (segment (start 137.1462 93.5536) (end 137.1462 91.6232) (width 0.127) (layer "F.Cu") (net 6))
 (via (at 124.5478 99.1162) (size 0.25) (drill 0.15) (layers "F.Cu" "B.Cu") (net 6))
 (via (at 122.719 96.5082) (size 0.25) (drill 0.15) (layers "F.Cu" "B.Cu") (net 6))
 (via (at 137.9082 94.1632) (size 0.25) (drill 0.15) (layers "F.Cu" "B.Cu") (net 6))
 (via (at 147.759 97.2112) (size 0.25) (drill 0.15) (layers "F.Cu" "B.Cu") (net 6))
 (segment (start 122.719 96.5082) (end 123.8366 97.6258) (width 0.127) (layer "B.Cu") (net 6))
 (segment (start 144.711 94.1632) (end 147.759 97.2112) (width 0.127) (layer "B.Cu") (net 6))
 (segment (start 122.719 96.5082) (end 125.064 94.1632) (width 0.127) (layer "B.Cu") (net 6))
 (segment (start 123.8366 98.405) (end 124.5478 99.1162) (width 0.127) (layer "B.Cu") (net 6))
 (segment (start 125.064 94.1632) (end 144.711 94.1632) (width 0.127) (layer "B.Cu") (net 6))
 (segment (start 123.8366 97.6258) (end 123.8366 98.405) (width 0.127) (layer "B.Cu") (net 6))
 (segment (start 136.0032 93.0202) (end 134.6062 91.6232) (width 0.127) (layer "F.Cu") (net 4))
 (segment (start 147.845 96.1542) (end 147.759 96.0682) (width 0.127) (layer "F.Cu") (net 4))
 (segment (start 121.1702 96.85) (end 121.1758 96.8556) (width 0.127) (layer "F.Cu") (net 4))
 (segment (start 149.537 96.1542) (end 147.845 96.1542) (width 0.127) (layer "F.Cu") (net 4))
 (segment (start 124.1717 96.8556) (end 124.4755 96.8556) (width 0.127) (layer "F.Cu") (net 4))
 (segment (start 125.3093 98.1122) (end 125.3093 97.6894) (width 0.127) (layer "F.Cu") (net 4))
 (segment (start 124.4462 94.1632) (end 124.4462 96.0936) (width 0.127) (layer "F.Cu") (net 4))
 (segment (start 124.4462 96.0936) (end 123.6842 96.8556) (width 0.127) (layer "F.Cu") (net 4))
 (segment (start 121.1758 96.8556) (end 124.1717 96.8556) (width 0.127) (layer "F.Cu") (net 4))
 (segment (start 124.4755 96.8556) (end 125.3093 97.6894) (width 0.127) (layer "F.Cu") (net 4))
 (via (at 147.759 96.0682) (size 0.25) (drill 0.15) (layers "F.Cu" "B.Cu") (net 4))
 (via (at 124.4462 94.1632) (size 0.25) (drill 0.15) (layers "F.Cu" "B.Cu") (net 4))
 (via (at 136.0032 93.0202) (size 0.25) (drill 0.15) (layers "F.Cu" "B.Cu") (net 4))
 (segment (start 124.4462 94.1632) (end 125.5892 93.0202) (width 0.127) (layer "B.Cu") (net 4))
 (segment (start 125.5892 93.0202) (end 144.711 93.0202) (width 0.127) (layer "B.Cu") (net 4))
 (segment (start 144.711 93.0202) (end 147.759 96.0682) (width 0.127) (layer "B.Cu") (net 4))
 (segment (start 119.6202 96.5) (end 119.6202 96.85) (width 0.127) (layer "F.Cu") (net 19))
 (segment (start 124.2136 98.6122) (end 123.8366 98.9892) (width 0.127) (layer "F.Cu") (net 3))
 (segment (start 123.8366 99.7068) (end 125.151 101.0212) (width 0.127) (layer "F.Cu") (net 3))
 (segment (start 123.8366 98.9892) (end 123.8366 99.7068) (width 0.127) (layer "F.Cu") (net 3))
 (segment (start 125.3093 98.6122) (end 124.2136 98.6122) (width 0.127) (layer "F.Cu") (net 3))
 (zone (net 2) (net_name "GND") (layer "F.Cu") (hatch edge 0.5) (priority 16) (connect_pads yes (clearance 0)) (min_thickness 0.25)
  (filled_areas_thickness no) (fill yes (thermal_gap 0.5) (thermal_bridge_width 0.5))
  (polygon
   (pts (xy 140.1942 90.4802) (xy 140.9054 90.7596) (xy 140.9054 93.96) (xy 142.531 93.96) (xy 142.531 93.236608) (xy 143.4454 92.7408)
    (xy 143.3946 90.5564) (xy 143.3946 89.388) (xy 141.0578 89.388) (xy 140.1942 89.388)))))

